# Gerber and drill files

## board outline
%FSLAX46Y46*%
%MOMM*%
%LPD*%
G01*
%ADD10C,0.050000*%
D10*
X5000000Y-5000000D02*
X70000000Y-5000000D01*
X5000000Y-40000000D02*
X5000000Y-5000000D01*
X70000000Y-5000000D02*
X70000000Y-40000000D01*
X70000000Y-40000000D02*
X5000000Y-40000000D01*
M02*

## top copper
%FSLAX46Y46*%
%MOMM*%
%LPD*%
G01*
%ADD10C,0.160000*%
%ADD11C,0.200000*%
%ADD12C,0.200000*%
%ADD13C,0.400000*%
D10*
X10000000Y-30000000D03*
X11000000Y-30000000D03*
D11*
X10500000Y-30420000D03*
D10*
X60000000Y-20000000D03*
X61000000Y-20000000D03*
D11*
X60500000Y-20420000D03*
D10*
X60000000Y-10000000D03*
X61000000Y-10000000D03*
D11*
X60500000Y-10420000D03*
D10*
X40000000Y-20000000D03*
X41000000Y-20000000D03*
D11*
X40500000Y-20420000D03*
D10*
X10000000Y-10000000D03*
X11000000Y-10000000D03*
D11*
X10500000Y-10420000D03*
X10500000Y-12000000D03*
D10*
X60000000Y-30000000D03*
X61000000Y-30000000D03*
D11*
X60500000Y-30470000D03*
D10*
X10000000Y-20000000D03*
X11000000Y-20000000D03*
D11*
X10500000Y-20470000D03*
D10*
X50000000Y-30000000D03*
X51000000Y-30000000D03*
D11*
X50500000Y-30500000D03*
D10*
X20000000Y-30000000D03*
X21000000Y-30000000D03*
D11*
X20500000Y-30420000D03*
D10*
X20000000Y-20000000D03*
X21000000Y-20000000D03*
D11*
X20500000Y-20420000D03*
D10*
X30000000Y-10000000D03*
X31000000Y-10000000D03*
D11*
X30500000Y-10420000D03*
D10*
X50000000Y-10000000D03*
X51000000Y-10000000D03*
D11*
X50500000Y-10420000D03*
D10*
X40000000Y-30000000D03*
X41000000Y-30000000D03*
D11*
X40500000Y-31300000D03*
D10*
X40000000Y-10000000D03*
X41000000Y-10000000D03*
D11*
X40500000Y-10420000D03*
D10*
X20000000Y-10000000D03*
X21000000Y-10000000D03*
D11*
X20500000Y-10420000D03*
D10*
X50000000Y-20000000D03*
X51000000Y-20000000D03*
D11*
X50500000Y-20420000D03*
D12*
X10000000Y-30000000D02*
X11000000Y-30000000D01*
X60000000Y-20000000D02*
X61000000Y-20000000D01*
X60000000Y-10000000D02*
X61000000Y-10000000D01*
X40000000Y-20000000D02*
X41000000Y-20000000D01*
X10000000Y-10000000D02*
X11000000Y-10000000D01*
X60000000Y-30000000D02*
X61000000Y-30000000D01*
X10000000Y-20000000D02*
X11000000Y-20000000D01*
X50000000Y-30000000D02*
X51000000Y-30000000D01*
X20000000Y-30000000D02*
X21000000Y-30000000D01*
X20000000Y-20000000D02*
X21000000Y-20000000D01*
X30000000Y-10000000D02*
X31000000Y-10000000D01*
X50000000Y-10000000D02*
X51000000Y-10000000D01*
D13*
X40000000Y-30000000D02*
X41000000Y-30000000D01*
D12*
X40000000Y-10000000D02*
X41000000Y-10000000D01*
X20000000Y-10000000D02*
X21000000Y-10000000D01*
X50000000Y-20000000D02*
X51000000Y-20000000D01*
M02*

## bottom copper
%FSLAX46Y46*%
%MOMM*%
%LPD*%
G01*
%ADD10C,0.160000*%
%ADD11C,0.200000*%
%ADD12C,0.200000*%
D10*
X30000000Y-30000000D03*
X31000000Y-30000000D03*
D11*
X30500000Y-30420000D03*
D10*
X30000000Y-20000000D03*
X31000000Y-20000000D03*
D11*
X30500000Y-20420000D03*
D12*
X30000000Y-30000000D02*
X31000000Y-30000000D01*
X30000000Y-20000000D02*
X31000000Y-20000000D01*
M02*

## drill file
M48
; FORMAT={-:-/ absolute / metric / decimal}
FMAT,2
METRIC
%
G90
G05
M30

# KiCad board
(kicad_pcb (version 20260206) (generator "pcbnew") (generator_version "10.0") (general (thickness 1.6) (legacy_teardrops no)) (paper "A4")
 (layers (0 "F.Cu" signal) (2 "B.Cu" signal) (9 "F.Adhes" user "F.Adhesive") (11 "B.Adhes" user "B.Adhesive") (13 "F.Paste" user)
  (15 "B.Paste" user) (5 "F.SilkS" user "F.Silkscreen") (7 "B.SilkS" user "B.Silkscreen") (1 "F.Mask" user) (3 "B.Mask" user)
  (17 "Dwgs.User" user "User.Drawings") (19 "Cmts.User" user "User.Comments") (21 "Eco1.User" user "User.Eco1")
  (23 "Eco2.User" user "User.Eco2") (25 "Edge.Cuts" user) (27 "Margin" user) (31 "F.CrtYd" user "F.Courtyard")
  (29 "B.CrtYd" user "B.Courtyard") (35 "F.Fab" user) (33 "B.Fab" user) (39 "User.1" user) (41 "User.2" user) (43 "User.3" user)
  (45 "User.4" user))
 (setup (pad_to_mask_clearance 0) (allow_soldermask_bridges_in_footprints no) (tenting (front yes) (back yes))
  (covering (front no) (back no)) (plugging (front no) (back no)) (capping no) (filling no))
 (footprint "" (layer "F.Cu") (at 10 30)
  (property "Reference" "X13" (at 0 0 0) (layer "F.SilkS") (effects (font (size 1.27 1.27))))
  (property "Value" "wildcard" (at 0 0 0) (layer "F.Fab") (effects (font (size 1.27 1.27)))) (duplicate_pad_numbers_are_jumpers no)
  (pad "1" smd circle (at 0 0) (size 0.16 0.16) (layers "F.Cu") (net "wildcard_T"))
  (pad "2" smd circle (at 1 0) (size 0.16 0.16) (layers "F.Cu") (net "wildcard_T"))
  (pad "3" smd circle (at 0.5 0.42) (size 0.2 0.2) (layers "F.Cu") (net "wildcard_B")))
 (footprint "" (layer "F.Cu") (at 60 20)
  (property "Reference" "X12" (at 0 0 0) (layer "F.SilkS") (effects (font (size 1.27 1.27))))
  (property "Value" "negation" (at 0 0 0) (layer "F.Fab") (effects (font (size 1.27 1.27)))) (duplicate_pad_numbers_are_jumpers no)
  (pad "1" smd circle (at 0 0) (size 0.16 0.16) (layers "F.Cu") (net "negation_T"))
  (pad "2" smd circle (at 1 0) (size 0.16 0.16) (layers "F.Cu") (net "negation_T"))
  (pad "3" smd circle (at 0.5 0.42) (size 0.2 0.2) (layers "F.Cu") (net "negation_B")))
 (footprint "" (layer "F.Cu") (at 60 10)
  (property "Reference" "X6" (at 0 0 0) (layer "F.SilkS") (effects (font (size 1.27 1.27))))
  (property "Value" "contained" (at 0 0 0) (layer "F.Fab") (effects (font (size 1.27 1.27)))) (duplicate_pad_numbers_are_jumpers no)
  (pad "1" smd circle (at 0 0) (size 0.16 0.16) (layers "F.Cu") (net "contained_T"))
  (pad "2" smd circle (at 1 0) (size 0.16 0.16) (layers "F.Cu") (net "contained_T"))
  (pad "3" smd circle (at 0.5 0.42) (size 0.2 0.2) (layers "F.Cu") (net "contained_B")))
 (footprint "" (layer "F.Cu") (at 40 20)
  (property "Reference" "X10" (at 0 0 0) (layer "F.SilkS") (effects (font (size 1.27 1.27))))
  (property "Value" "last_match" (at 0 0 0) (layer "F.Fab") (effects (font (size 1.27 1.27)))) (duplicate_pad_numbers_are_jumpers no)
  (pad "1" smd circle (at 0 0) (size 0.16 0.16) (layers "F.Cu") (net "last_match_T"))
  (pad "2" smd circle (at 1 0) (size 0.16 0.16) (layers "F.Cu") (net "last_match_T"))
  (pad "3" smd circle (at 0.5 0.42) (size 0.2 0.2) (layers "F.Cu") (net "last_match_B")))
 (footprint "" (layer "F.Cu") (at 10 10)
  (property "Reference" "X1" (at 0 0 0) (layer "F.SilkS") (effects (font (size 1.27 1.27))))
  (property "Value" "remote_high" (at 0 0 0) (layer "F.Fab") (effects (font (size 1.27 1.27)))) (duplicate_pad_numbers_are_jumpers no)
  (pad "1" smd circle (at 0 0) (size 0.16 0.16) (layers "F.Cu") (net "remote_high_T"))
  (pad "2" smd circle (at 1 0) (size 0.16 0.16) (layers "F.Cu") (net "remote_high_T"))
  (pad "3" smd circle (at 0.5 0.42) (size 0.2 0.2) (layers "F.Cu") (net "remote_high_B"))
  (pad "4" smd circle (at 0.5 2) (size 0.2 0.2) (layers "F.Cu") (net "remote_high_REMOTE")))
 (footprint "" (layer "F.Cu") (at 60 30)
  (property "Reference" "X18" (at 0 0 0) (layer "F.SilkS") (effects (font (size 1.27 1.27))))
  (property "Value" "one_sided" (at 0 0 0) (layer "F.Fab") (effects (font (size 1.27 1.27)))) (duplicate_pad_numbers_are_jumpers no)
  (pad "1" smd circle (at 0 0) (size 0.16 0.16) (layers "F.Cu") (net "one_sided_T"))
  (pad "2" smd circle (at 1 0) (size 0.16 0.16) (layers "F.Cu") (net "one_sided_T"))
  (pad "3" smd circle (at 0.5 0.47) (size 0.2 0.2) (layers "F.Cu") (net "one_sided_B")))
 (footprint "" (layer "F.Cu") (at 10 20)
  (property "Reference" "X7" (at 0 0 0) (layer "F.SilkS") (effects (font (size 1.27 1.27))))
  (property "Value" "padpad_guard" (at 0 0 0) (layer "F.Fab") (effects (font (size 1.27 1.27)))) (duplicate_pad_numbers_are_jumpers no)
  (pad "1" smd circle (at 0 0) (size 0.16 0.16) (layers "F.Cu") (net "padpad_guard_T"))
  (pad "2" smd circle (at 1 0) (size 0.16 0.16) (layers "F.Cu") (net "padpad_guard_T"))
  (pad "3" smd circle (at 0.5 0.47) (size 0.2 0.2) (layers "F.Cu") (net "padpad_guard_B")))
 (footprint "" (layer "F.Cu") (at 50 30)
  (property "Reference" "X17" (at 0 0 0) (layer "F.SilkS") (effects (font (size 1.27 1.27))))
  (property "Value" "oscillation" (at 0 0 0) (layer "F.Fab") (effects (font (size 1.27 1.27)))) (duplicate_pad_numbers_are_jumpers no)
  (pad "1" smd circle (at 0 0) (size 0.16 0.16) (layers "F.Cu") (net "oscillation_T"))
  (pad "2" smd circle (at 1 0) (size 0.16 0.16) (layers "F.Cu") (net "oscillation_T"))
  (pad "3" smd circle (at 0.5 0.5) (size 0.2 0.2) (layers "F.Cu") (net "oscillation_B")))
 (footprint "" (layer "F.Cu") (at 20 30)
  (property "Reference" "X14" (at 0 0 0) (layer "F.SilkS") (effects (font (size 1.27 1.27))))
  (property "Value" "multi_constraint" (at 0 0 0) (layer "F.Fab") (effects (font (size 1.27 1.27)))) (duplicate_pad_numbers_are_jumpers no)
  (pad "1" smd circle (at 0 0) (size 0.16 0.16) (layers "F.Cu") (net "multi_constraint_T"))
  (pad "2" smd circle (at 1 0) (size 0.16 0.16) (layers "F.Cu") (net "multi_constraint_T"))
  (pad "3" smd circle (at 0.5 0.42) (size 0.2 0.2) (layers "F.Cu") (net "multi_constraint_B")))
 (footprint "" (layer "F.Cu") (at 30 30)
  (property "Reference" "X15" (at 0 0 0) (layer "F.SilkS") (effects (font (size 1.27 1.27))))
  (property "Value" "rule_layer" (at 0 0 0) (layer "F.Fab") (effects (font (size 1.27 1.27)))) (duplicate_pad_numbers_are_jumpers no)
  (pad "1" smd circle (at 0 0) (size 0.16 0.16) (layers "B.Cu") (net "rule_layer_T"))
  (pad "2" smd circle (at 1 0) (size 0.16 0.16) (layers "B.Cu") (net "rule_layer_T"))
  (pad "3" smd circle (at 0.5 0.42) (size 0.2 0.2) (layers "B.Cu") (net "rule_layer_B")))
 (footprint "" (layer "F.Cu") (at 20 20)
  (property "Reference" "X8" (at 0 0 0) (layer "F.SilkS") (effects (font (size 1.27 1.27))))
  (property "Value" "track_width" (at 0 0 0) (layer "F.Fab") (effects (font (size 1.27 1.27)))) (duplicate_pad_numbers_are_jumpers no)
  (pad "1" smd circle (at 0 0) (size 0.16 0.16) (layers "F.Cu") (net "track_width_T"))
  (pad "2" smd circle (at 1 0) (size 0.16 0.16) (layers "F.Cu") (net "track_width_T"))
  (pad "3" smd circle (at 0.5 0.42) (size 0.2 0.2) (layers "F.Cu") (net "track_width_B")))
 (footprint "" (layer "F.Cu") (at 30 10)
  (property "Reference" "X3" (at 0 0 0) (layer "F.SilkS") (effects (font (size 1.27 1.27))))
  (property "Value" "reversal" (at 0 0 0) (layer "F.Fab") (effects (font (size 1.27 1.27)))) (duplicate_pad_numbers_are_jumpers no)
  (pad "1" smd circle (at 0 0) (size 0.16 0.16) (layers "F.Cu") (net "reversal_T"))
  (pad "2" smd circle (at 1 0) (size 0.16 0.16) (layers "F.Cu") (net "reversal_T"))
  (pad "3" smd circle (at 0.5 0.42) (size 0.2 0.2) (layers "F.Cu") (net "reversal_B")))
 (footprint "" (layer "F.Cu") (at 50 10)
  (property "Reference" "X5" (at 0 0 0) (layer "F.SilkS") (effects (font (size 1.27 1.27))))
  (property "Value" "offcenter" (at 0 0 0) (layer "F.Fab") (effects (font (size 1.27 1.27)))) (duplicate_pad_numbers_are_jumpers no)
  (pad "1" smd circle (at 0 0) (size 0.16 0.16) (layers "F.Cu") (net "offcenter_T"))
  (pad "2" smd circle (at 1 0) (size 0.16 0.16) (layers "F.Cu") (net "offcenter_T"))
  (pad "3" smd circle (at 0.5 0.42) (size 0.2 0.2) (layers "F.Cu") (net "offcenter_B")))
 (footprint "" (layer "F.Cu") (at 40 30)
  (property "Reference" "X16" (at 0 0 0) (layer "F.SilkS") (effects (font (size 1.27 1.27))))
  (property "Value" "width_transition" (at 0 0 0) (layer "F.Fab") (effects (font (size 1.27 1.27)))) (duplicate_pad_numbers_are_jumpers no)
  (pad "1" smd circle (at 0 0) (size 0.16 0.16) (layers "F.Cu") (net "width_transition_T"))
  (pad "2" smd circle (at 1 0) (size 0.16 0.16) (layers "F.Cu") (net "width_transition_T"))
  (pad "3" smd circle (at 0.5 1.3) (size 0.2 0.2) (layers "F.Cu") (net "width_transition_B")))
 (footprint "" (layer "F.Cu") (at 30 20)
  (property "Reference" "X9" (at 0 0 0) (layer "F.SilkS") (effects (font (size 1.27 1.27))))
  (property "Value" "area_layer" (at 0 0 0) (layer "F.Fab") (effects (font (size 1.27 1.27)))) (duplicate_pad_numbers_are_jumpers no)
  (pad "1" smd circle (at 0 0) (size 0.16 0.16) (layers "B.Cu") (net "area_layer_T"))
  (pad "2" smd circle (at 1 0) (size 0.16 0.16) (layers "B.Cu") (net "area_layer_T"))
  (pad "3" smd circle (at 0.5 0.42) (size 0.2 0.2) (layers "B.Cu") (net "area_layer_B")))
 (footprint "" (layer "F.Cu") (at 40 10)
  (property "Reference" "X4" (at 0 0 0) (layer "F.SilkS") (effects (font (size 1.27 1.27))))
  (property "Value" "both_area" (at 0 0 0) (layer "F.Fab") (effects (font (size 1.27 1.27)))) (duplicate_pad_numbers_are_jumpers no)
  (pad "1" smd circle (at 0 0) (size 0.16 0.16) (layers "F.Cu") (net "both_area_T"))
  (pad "2" smd circle (at 1 0) (size 0.16 0.16) (layers "F.Cu") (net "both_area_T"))
  (pad "3" smd circle (at 0.5 0.42) (size 0.2 0.2) (layers "F.Cu") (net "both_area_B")))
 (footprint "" (layer "F.Cu") (at 20 10)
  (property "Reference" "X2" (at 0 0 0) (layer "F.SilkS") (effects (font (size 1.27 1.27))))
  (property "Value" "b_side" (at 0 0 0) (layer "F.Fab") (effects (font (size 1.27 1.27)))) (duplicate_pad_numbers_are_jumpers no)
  (pad "1" smd circle (at 0 0) (size 0.16 0.16) (layers "F.Cu") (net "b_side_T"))
  (pad "2" smd circle (at 1 0) (size 0.16 0.16) (layers "F.Cu") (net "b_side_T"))
  (pad "3" smd circle (at 0.5 0.42) (size 0.2 0.2) (layers "F.Cu") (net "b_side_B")))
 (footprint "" (layer "F.Cu") (at 50 20)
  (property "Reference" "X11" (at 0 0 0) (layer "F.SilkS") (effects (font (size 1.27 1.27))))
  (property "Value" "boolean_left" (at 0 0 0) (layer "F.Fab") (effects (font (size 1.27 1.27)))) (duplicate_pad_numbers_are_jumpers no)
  (pad "1" smd circle (at 0 0) (size 0.16 0.16) (layers "F.Cu") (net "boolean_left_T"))
  (pad "2" smd circle (at 1 0) (size 0.16 0.16) (layers "F.Cu") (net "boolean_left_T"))
  (pad "3" smd circle (at 0.5 0.42) (size 0.2 0.2) (layers "F.Cu") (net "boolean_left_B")))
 (gr_line (start 5 5) (end 70 5) (stroke (width 0.05) (type default)) (layer "Edge.Cuts"))
 (gr_line (start 5 40) (end 5 5) (stroke (width 0.05) (type default)) (layer "Edge.Cuts"))
 (gr_line (start 70 5) (end 70 40) (stroke (width 0.05) (type default)) (layer "Edge.Cuts"))
 (gr_line (start 70 40) (end 5 40) (stroke (width 0.05) (type default)) (layer "Edge.Cuts"))
 (segment (start 10 30) (end 11 30) (width 0.2) (layer "F.Cu") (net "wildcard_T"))
 (segment (start 60 20) (end 61 20) (width 0.2) (layer "F.Cu") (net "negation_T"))
 (segment (start 60 10) (end 61 10) (width 0.2) (layer "F.Cu") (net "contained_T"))
 (segment (start 40 20) (end 41 20) (width 0.2) (layer "F.Cu") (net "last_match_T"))
 (segment (start 10 10) (end 11 10) (width 0.2) (layer "F.Cu") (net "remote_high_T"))
 (segment (start 60 30) (end 61 30) (width 0.2) (layer "F.Cu") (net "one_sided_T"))
 (segment (start 10 20) (end 11 20) (width 0.2) (layer "F.Cu") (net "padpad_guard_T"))
 (segment (start 50 30) (end 51 30) (width 0.2) (layer "F.Cu") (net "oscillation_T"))
 (segment (start 20 30) (end 21 30) (width 0.2) (layer "F.Cu") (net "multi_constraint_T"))
 (segment (start 30 30) (end 31 30) (width 0.2) (layer "B.Cu") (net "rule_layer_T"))
 (segment (start 20 20) (end 21 20) (width 0.2) (layer "F.Cu") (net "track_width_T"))
 (segment (start 30 10) (end 31 10) (width 0.2) (layer "F.Cu") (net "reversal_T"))
 (segment (start 50 10) (end 51 10) (width 0.2) (layer "F.Cu") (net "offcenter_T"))
 (segment (start 40 30) (end 41 30) (width 0.4) (layer "F.Cu") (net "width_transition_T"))
 (segment (start 30 20) (end 31 20) (width 0.2) (layer "B.Cu") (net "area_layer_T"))
 (segment (start 40 10) (end 41 10) (width 0.2) (layer "F.Cu") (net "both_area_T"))
 (segment (start 20 10) (end 21 10) (width 0.2) (layer "F.Cu") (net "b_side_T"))
 (segment (start 50 20) (end 51 20) (width 0.2) (layer "F.Cu") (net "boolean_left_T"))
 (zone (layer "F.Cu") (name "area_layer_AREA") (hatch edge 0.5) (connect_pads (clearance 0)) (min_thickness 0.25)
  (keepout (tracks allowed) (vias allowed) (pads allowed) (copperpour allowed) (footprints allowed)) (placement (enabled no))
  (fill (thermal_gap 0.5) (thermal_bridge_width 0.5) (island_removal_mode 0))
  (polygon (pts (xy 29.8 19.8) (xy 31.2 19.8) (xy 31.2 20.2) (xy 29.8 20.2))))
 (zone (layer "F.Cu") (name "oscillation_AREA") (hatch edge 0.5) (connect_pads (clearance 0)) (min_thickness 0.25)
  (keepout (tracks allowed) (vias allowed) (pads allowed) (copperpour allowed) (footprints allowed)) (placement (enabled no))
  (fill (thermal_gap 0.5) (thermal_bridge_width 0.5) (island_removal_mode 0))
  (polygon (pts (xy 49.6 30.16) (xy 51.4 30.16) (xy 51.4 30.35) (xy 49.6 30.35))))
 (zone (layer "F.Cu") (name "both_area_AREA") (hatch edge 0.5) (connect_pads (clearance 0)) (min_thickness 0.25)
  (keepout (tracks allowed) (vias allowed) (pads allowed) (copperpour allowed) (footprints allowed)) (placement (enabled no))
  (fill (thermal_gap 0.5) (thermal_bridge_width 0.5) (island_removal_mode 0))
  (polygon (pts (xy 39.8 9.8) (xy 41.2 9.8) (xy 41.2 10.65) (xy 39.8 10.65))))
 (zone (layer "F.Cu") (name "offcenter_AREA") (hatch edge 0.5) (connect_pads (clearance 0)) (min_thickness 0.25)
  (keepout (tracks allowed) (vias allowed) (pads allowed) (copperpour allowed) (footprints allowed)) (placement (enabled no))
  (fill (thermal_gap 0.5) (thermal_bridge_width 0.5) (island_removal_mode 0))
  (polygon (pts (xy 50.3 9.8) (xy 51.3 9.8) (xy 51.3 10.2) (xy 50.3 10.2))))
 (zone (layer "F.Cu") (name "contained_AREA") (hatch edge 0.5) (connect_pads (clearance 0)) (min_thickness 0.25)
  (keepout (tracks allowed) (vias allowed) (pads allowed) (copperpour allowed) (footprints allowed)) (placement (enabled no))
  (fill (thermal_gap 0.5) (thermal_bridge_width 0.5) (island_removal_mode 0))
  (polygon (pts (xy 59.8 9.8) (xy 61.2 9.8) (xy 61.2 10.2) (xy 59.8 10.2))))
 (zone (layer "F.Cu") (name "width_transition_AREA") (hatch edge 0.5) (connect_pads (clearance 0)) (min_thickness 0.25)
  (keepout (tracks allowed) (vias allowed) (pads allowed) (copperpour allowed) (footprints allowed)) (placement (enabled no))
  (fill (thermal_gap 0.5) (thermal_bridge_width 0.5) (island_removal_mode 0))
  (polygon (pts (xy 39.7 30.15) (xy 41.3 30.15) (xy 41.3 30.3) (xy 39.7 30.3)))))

